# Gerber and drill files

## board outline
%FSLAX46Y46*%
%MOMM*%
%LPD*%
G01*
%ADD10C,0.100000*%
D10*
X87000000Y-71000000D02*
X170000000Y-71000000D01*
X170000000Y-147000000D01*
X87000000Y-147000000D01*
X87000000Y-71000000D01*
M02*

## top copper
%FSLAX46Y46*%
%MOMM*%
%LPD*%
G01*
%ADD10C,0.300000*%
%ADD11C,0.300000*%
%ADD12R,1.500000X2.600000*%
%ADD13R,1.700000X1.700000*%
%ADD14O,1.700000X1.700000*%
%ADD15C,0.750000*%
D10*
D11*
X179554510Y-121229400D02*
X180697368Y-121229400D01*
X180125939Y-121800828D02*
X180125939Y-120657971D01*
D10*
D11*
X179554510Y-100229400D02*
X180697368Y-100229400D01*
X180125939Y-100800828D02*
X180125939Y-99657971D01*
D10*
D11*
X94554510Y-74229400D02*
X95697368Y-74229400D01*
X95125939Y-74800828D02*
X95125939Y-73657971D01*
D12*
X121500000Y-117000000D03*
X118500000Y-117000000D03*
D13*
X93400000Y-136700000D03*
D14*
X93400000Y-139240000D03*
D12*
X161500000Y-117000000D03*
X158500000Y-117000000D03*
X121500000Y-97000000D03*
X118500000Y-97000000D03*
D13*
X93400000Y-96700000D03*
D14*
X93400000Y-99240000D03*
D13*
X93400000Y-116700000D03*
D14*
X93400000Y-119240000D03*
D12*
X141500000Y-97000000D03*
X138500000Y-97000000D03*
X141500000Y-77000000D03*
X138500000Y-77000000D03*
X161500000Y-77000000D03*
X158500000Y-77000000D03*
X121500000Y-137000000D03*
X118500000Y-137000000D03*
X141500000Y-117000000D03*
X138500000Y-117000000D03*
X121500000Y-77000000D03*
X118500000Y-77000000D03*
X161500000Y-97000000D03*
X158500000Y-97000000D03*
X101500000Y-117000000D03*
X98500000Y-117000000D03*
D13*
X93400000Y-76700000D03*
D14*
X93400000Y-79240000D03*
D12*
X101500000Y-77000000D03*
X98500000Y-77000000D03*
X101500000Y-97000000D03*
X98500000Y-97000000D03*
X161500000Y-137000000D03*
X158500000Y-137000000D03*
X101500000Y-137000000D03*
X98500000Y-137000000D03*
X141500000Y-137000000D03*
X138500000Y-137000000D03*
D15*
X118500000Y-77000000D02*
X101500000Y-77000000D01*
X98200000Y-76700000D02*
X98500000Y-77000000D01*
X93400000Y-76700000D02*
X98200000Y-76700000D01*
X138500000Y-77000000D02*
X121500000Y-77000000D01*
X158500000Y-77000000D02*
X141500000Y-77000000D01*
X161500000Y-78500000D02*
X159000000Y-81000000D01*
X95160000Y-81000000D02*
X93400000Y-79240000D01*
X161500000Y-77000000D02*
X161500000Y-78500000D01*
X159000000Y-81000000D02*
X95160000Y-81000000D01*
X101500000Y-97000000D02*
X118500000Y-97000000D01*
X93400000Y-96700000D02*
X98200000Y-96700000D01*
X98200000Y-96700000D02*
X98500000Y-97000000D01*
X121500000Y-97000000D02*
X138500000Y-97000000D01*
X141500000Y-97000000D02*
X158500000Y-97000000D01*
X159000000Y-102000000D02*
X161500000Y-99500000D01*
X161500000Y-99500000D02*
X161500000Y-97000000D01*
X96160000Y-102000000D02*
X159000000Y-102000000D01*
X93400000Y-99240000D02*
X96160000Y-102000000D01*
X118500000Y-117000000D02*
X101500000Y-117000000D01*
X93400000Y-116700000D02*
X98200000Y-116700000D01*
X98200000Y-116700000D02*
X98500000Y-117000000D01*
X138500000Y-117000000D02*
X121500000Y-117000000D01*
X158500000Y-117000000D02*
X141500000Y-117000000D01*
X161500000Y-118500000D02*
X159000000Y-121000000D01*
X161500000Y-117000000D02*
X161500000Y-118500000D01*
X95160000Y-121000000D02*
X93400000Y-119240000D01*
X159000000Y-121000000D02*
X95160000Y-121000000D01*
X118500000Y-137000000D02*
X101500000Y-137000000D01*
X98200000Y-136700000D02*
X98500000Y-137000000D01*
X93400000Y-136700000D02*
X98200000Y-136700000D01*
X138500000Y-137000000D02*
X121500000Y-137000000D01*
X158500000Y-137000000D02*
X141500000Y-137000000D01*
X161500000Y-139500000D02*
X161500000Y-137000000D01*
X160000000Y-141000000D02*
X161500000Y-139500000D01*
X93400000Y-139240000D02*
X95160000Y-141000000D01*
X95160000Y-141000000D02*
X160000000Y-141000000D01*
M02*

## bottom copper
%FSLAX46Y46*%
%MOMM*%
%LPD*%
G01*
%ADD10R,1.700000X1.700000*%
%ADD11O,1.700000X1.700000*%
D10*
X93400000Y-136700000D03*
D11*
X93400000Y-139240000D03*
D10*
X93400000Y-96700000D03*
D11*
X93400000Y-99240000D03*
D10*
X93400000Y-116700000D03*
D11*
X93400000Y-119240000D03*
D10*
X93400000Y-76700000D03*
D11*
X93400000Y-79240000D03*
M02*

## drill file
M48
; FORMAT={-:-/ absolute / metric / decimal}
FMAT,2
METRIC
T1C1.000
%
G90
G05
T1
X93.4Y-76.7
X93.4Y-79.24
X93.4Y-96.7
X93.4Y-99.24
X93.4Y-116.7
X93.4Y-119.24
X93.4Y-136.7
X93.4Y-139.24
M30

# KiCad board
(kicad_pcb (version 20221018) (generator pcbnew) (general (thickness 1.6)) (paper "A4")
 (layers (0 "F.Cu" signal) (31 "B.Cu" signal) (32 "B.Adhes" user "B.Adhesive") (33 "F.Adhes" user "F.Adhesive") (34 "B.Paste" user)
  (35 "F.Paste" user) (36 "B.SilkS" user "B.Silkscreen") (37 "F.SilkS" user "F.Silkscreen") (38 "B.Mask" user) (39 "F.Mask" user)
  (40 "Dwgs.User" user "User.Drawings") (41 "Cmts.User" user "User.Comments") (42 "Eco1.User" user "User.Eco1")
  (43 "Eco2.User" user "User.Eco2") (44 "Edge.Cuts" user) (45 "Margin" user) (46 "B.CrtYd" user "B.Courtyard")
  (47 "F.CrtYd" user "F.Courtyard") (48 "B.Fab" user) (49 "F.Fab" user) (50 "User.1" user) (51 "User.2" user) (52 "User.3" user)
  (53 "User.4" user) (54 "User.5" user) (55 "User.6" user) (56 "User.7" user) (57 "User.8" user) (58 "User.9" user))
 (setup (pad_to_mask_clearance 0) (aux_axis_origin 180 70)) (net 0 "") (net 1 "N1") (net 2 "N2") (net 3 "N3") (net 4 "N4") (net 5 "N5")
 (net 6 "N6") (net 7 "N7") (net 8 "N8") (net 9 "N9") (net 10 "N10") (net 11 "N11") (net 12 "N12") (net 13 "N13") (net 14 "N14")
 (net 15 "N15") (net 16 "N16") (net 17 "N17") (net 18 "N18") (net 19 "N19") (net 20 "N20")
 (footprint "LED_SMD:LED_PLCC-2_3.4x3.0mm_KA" (layer "F.Cu") (at 120 117 180)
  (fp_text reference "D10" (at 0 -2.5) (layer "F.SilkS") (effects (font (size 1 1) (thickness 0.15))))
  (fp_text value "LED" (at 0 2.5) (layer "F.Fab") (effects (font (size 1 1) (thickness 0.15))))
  (pad "1" smd rect (at -1.5 0 180) (size 1.5 2.6) (layers "F.Cu" "F.Paste" "F.Mask") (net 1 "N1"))
  (pad "2" smd rect (at 1.5 0 180) (size 1.5 2.6) (layers "F.Cu" "F.Paste" "F.Mask") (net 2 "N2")))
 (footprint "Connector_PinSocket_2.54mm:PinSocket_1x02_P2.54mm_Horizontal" (layer "F.Cu") (at 93.4 136.7)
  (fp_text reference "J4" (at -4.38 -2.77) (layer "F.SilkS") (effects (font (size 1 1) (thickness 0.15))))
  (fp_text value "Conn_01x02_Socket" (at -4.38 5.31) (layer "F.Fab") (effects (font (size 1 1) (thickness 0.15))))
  (pad "1" thru_hole rect (at 0 0) (size 1.7 1.7) (drill 1) (layers "*.Cu" "*.Mask") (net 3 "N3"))
  (pad "2" thru_hole oval (at 0 2.54) (size 1.7 1.7) (drill 1) (layers "*.Cu" "*.Mask") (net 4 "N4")))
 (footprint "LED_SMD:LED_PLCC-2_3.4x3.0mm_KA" (layer "F.Cu") (at 160 117 180)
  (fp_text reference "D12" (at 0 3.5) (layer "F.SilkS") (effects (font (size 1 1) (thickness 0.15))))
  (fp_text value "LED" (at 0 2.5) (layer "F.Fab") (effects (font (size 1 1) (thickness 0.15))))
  (pad "1" smd rect (at -1.5 0 180) (size 1.5 2.6) (layers "F.Cu" "F.Paste" "F.Mask") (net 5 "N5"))
  (pad "2" smd rect (at 1.5 0 180) (size 1.5 2.6) (layers "F.Cu" "F.Paste" "F.Mask") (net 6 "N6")))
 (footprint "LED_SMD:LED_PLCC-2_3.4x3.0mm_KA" (layer "F.Cu") (at 120 97 180)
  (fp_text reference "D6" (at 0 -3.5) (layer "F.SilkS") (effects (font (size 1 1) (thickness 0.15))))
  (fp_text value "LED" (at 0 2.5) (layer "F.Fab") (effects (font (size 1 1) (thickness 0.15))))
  (pad "1" smd rect (at -1.5 0 180) (size 1.5 2.6) (layers "F.Cu" "F.Paste" "F.Mask") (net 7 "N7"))
  (pad "2" smd rect (at 1.5 0 180) (size 1.5 2.6) (layers "F.Cu" "F.Paste" "F.Mask") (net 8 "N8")))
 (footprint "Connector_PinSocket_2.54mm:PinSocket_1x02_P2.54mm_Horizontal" (layer "F.Cu") (at 93.4 96.7)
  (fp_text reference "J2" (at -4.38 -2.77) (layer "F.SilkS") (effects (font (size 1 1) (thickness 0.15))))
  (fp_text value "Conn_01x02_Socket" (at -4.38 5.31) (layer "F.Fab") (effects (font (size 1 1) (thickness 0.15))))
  (pad "1" thru_hole rect (at 0 0) (size 1.7 1.7) (drill 1) (layers "*.Cu" "*.Mask") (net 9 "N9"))
  (pad "2" thru_hole oval (at 0 2.54) (size 1.7 1.7) (drill 1) (layers "*.Cu" "*.Mask") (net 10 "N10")))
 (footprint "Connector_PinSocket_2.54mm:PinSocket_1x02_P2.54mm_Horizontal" (layer "F.Cu") (at 93.4 116.7)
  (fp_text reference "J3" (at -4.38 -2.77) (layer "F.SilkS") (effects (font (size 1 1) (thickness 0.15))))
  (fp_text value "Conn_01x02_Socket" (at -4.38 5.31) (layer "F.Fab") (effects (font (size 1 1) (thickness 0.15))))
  (pad "1" thru_hole rect (at 0 0) (size 1.7 1.7) (drill 1) (layers "*.Cu" "*.Mask") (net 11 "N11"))
  (pad "2" thru_hole oval (at 0 2.54) (size 1.7 1.7) (drill 1) (layers "*.Cu" "*.Mask") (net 5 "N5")))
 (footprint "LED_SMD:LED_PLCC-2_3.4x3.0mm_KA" (layer "F.Cu") (at 140 97 180)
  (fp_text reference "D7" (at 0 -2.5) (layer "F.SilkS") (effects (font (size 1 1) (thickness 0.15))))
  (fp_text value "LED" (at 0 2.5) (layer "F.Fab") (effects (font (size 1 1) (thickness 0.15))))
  (pad "1" smd rect (at -1.5 0 180) (size 1.5 2.6) (layers "F.Cu" "F.Paste" "F.Mask") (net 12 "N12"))
  (pad "2" smd rect (at 1.5 0 180) (size 1.5 2.6) (layers "F.Cu" "F.Paste" "F.Mask") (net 7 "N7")))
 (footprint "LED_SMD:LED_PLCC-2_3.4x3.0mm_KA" (layer "F.Cu") (at 140 77 180)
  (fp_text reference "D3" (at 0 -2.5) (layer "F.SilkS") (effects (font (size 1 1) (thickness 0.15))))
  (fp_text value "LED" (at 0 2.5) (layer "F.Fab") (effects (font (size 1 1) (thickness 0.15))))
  (pad "1" smd rect (at -1.5 0 180) (size 1.5 2.6) (layers "F.Cu" "F.Paste" "F.Mask") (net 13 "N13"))
  (pad "2" smd rect (at 1.5 0 180) (size 1.5 2.6) (layers "F.Cu" "F.Paste" "F.Mask") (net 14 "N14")))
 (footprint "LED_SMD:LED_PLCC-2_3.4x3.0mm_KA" (layer "F.Cu") (at 160 77 180)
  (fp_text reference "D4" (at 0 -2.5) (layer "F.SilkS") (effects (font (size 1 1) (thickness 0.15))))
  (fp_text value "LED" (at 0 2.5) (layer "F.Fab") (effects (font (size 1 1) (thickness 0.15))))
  (pad "1" smd rect (at -1.5 0 180) (size 1.5 2.6) (layers "F.Cu" "F.Paste" "F.Mask") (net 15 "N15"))
  (pad "2" smd rect (at 1.5 0 180) (size 1.5 2.6) (layers "F.Cu" "F.Paste" "F.Mask") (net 13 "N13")))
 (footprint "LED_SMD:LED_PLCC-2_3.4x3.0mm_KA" (layer "F.Cu") (at 120 137 180)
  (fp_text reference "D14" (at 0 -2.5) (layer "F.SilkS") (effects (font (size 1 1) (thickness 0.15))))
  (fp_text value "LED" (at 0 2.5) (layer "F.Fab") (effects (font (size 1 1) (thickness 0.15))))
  (pad "1" smd rect (at -1.5 0 180) (size 1.5 2.6) (layers "F.Cu" "F.Paste" "F.Mask") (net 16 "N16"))
  (pad "2" smd rect (at 1.5 0 180) (size 1.5 2.6) (layers "F.Cu" "F.Paste" "F.Mask") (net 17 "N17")))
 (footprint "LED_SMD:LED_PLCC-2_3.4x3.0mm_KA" (layer "F.Cu") (at 140 117 180)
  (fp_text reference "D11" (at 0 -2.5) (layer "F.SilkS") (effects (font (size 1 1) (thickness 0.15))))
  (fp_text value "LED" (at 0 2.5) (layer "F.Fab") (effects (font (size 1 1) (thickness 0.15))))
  (pad "1" smd rect (at -1.5 0 180) (size 1.5 2.6) (layers "F.Cu" "F.Paste" "F.Mask") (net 6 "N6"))
  (pad "2" smd rect (at 1.5 0 180) (size 1.5 2.6) (layers "F.Cu" "F.Paste" "F.Mask") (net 1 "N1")))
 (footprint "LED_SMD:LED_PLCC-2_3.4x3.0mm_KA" (layer "F.Cu") (at 120 77 180)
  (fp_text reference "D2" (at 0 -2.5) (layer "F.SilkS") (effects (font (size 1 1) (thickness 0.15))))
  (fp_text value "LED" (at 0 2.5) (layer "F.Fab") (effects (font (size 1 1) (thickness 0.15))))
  (pad "1" smd rect (at -1.5 0 180) (size 1.5 2.6) (layers "F.Cu" "F.Paste" "F.Mask") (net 14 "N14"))
  (pad "2" smd rect (at 1.5 0 180) (size 1.5 2.6) (layers "F.Cu" "F.Paste" "F.Mask") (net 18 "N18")))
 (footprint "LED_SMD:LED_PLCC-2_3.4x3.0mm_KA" (layer "F.Cu") (at 160 97 180)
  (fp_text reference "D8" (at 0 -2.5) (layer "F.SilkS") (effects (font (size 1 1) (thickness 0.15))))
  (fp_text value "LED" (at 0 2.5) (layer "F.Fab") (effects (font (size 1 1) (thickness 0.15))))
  (pad "1" smd rect (at -1.5 0 180) (size 1.5 2.6) (layers "F.Cu" "F.Paste" "F.Mask") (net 10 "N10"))
  (pad "2" smd rect (at 1.5 0 180) (size 1.5 2.6) (layers "F.Cu" "F.Paste" "F.Mask") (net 12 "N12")))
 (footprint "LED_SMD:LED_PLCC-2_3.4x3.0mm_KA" (layer "F.Cu") (at 100 117 180)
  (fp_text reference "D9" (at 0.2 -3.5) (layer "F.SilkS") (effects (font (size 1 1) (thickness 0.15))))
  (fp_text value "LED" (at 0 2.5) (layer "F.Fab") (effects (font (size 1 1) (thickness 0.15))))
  (pad "1" smd rect (at -1.5 0 180) (size 1.5 2.6) (layers "F.Cu" "F.Paste" "F.Mask") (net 2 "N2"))
  (pad "2" smd rect (at 1.5 0 180) (size 1.5 2.6) (layers "F.Cu" "F.Paste" "F.Mask") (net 11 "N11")))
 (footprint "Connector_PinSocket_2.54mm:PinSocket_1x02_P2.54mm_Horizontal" (layer "F.Cu") (at 93.4 76.7)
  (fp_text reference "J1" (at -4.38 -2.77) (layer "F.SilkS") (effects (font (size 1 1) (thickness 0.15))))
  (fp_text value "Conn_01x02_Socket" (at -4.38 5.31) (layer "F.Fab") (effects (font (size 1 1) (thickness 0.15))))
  (pad "1" thru_hole rect (at 0 0) (size 1.7 1.7) (drill 1) (layers "*.Cu" "*.Mask") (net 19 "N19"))
  (pad "2" thru_hole oval (at 0 2.54) (size 1.7 1.7) (drill 1) (layers "*.Cu" "*.Mask") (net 15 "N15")))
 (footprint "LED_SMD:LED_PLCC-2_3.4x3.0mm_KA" (layer "F.Cu") (at 100 77 180)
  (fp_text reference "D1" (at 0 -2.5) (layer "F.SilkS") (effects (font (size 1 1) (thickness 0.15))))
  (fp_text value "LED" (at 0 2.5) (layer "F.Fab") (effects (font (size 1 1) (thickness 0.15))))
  (pad "1" smd rect (at -1.5 0 180) (size 1.5 2.6) (layers "F.Cu" "F.Paste" "F.Mask") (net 18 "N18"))
  (pad "2" smd rect (at 1.5 0 180) (size 1.5 2.6) (layers "F.Cu" "F.Paste" "F.Mask") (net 19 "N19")))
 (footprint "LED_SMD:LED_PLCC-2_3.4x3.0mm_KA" (layer "F.Cu") (at 100 97 180)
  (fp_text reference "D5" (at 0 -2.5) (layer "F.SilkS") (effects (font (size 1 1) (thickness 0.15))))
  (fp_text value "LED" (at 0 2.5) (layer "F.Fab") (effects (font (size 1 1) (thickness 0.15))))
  (pad "1" smd rect (at -1.5 0 180) (size 1.5 2.6) (layers "F.Cu" "F.Paste" "F.Mask") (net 8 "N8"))
  (pad "2" smd rect (at 1.5 0 180) (size 1.5 2.6) (layers "F.Cu" "F.Paste" "F.Mask") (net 9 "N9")))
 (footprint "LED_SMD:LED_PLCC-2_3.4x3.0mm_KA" (layer "F.Cu") (at 160 137 180)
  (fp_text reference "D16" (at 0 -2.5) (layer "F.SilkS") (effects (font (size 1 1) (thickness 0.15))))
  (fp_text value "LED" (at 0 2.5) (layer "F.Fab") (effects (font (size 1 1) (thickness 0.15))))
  (pad "1" smd rect (at -1.5 0 180) (size 1.5 2.6) (layers "F.Cu" "F.Paste" "F.Mask") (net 4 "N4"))
  (pad "2" smd rect (at 1.5 0 180) (size 1.5 2.6) (layers "F.Cu" "F.Paste" "F.Mask") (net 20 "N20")))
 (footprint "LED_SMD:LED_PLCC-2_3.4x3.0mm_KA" (layer "F.Cu") (at 100 137 180)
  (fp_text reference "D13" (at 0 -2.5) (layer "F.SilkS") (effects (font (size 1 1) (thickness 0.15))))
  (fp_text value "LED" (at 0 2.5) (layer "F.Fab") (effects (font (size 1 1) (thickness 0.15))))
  (pad "1" smd rect (at -1.5 0 180) (size 1.5 2.6) (layers "F.Cu" "F.Paste" "F.Mask") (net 17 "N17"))
  (pad "2" smd rect (at 1.5 0 180) (size 1.5 2.6) (layers "F.Cu" "F.Paste" "F.Mask") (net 3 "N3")))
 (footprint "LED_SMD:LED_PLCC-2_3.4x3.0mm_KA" (layer "F.Cu") (at 140 137 180)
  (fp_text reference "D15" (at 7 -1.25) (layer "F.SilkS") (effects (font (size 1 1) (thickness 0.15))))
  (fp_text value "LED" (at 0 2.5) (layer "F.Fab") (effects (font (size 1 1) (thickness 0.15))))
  (pad "1" smd rect (at -1.5 0 180) (size 1.5 2.6) (layers "F.Cu" "F.Paste" "F.Mask") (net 20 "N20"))
  (pad "2" smd rect (at 1.5 0 180) (size 1.5 2.6) (layers "F.Cu" "F.Paste" "F.Mask") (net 16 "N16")))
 (gr_rect (start 87 71) (end 170 147) (stroke (width 0.1) (type default)) (fill none) (layer "Edge.Cuts"))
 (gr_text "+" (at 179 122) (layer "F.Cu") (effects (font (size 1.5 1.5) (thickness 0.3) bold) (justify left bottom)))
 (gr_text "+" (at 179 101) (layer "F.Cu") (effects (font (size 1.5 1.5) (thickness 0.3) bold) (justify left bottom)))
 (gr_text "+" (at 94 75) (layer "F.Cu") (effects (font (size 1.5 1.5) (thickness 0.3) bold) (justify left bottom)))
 (segment (start 118.5 77) (end 101.5 77) (width 0.75) (layer "F.Cu") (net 18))
 (segment (start 98.2 76.7) (end 98.5 77) (width 0.75) (layer "F.Cu") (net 19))
 (segment (start 93.4 76.7) (end 98.2 76.7) (width 0.75) (layer "F.Cu") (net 19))
 (segment (start 138.5 77) (end 121.5 77) (width 0.75) (layer "F.Cu") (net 14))
 (segment (start 158.5 77) (end 141.5 77) (width 0.75) (layer "F.Cu") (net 13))
 (segment (start 161.5 78.5) (end 159 81) (width 0.75) (layer "F.Cu") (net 15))
 (segment (start 95.16 81) (end 93.4 79.24) (width 0.75) (layer "F.Cu") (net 15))
 (segment (start 161.5 77) (end 161.5 78.5) (width 0.75) (layer "F.Cu") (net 15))
 (segment (start 159 81) (end 95.16 81) (width 0.75) (layer "F.Cu") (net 15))
 (segment (start 101.5 97) (end 118.5 97) (width 0.75) (layer "F.Cu") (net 8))
 (segment (start 93.4 96.7) (end 98.2 96.7) (width 0.75) (layer "F.Cu") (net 9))
 (segment (start 98.2 96.7) (end 98.5 97) (width 0.75) (layer "F.Cu") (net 9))
 (segment (start 121.5 97) (end 138.5 97) (width 0.75) (layer "F.Cu") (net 7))
 (segment (start 141.5 97) (end 158.5 97) (width 0.75) (layer "F.Cu") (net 12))
 (segment (start 159 102) (end 161.5 99.5) (width 0.75) (layer "F.Cu") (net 10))
 (segment (start 161.5 99.5) (end 161.5 97) (width 0.75) (layer "F.Cu") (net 10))
 (segment (start 96.16 102) (end 159 102) (width 0.75) (layer "F.Cu") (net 10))
 (segment (start 93.4 99.24) (end 96.16 102) (width 0.75) (layer "F.Cu") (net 10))
 (segment (start 118.5 117) (end 101.5 117) (width 0.75) (layer "F.Cu") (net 2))
 (segment (start 93.4 116.7) (end 98.2 116.7) (width 0.75) (layer "F.Cu") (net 11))
 (segment (start 98.2 116.7) (end 98.5 117) (width 0.75) (layer "F.Cu") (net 11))
 (segment (start 138.5 117) (end 121.5 117) (width 0.75) (layer "F.Cu") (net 1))
 (segment (start 158.5 117) (end 141.5 117) (width 0.75) (layer "F.Cu") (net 6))
 (segment (start 161.5 118.5) (end 159 121) (width 0.75) (layer "F.Cu") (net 5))
 (segment (start 161.5 117) (end 161.5 118.5) (width 0.75) (layer "F.Cu") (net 5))
 (segment (start 95.16 121) (end 93.4 119.24) (width 0.75) (layer "F.Cu") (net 5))
 (segment (start 159 121) (end 95.16 121) (width 0.75) (layer "F.Cu") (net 5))
 (segment (start 118.5 137) (end 101.5 137) (width 0.75) (layer "F.Cu") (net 17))
 (segment (start 98.2 136.7) (end 98.5 137) (width 0.75) (layer "F.Cu") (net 3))
 (segment (start 93.4 136.7) (end 98.2 136.7) (width 0.75) (layer "F.Cu") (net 3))
 (segment (start 138.5 137) (end 121.5 137) (width 0.75) (layer "F.Cu") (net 16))
 (segment (start 158.5 137) (end 141.5 137) (width 0.75) (layer "F.Cu") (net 20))
 (segment (start 161.5 139.5) (end 161.5 137) (width 0.75) (layer "F.Cu") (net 4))
 (segment (start 160 141) (end 161.5 139.5) (width 0.75) (layer "F.Cu") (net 4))
 (segment (start 93.4 139.24) (end 95.16 141) (width 0.75) (layer "F.Cu") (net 4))
 (segment (start 95.16 141) (end 160 141) (width 0.75) (layer "F.Cu") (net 4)))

